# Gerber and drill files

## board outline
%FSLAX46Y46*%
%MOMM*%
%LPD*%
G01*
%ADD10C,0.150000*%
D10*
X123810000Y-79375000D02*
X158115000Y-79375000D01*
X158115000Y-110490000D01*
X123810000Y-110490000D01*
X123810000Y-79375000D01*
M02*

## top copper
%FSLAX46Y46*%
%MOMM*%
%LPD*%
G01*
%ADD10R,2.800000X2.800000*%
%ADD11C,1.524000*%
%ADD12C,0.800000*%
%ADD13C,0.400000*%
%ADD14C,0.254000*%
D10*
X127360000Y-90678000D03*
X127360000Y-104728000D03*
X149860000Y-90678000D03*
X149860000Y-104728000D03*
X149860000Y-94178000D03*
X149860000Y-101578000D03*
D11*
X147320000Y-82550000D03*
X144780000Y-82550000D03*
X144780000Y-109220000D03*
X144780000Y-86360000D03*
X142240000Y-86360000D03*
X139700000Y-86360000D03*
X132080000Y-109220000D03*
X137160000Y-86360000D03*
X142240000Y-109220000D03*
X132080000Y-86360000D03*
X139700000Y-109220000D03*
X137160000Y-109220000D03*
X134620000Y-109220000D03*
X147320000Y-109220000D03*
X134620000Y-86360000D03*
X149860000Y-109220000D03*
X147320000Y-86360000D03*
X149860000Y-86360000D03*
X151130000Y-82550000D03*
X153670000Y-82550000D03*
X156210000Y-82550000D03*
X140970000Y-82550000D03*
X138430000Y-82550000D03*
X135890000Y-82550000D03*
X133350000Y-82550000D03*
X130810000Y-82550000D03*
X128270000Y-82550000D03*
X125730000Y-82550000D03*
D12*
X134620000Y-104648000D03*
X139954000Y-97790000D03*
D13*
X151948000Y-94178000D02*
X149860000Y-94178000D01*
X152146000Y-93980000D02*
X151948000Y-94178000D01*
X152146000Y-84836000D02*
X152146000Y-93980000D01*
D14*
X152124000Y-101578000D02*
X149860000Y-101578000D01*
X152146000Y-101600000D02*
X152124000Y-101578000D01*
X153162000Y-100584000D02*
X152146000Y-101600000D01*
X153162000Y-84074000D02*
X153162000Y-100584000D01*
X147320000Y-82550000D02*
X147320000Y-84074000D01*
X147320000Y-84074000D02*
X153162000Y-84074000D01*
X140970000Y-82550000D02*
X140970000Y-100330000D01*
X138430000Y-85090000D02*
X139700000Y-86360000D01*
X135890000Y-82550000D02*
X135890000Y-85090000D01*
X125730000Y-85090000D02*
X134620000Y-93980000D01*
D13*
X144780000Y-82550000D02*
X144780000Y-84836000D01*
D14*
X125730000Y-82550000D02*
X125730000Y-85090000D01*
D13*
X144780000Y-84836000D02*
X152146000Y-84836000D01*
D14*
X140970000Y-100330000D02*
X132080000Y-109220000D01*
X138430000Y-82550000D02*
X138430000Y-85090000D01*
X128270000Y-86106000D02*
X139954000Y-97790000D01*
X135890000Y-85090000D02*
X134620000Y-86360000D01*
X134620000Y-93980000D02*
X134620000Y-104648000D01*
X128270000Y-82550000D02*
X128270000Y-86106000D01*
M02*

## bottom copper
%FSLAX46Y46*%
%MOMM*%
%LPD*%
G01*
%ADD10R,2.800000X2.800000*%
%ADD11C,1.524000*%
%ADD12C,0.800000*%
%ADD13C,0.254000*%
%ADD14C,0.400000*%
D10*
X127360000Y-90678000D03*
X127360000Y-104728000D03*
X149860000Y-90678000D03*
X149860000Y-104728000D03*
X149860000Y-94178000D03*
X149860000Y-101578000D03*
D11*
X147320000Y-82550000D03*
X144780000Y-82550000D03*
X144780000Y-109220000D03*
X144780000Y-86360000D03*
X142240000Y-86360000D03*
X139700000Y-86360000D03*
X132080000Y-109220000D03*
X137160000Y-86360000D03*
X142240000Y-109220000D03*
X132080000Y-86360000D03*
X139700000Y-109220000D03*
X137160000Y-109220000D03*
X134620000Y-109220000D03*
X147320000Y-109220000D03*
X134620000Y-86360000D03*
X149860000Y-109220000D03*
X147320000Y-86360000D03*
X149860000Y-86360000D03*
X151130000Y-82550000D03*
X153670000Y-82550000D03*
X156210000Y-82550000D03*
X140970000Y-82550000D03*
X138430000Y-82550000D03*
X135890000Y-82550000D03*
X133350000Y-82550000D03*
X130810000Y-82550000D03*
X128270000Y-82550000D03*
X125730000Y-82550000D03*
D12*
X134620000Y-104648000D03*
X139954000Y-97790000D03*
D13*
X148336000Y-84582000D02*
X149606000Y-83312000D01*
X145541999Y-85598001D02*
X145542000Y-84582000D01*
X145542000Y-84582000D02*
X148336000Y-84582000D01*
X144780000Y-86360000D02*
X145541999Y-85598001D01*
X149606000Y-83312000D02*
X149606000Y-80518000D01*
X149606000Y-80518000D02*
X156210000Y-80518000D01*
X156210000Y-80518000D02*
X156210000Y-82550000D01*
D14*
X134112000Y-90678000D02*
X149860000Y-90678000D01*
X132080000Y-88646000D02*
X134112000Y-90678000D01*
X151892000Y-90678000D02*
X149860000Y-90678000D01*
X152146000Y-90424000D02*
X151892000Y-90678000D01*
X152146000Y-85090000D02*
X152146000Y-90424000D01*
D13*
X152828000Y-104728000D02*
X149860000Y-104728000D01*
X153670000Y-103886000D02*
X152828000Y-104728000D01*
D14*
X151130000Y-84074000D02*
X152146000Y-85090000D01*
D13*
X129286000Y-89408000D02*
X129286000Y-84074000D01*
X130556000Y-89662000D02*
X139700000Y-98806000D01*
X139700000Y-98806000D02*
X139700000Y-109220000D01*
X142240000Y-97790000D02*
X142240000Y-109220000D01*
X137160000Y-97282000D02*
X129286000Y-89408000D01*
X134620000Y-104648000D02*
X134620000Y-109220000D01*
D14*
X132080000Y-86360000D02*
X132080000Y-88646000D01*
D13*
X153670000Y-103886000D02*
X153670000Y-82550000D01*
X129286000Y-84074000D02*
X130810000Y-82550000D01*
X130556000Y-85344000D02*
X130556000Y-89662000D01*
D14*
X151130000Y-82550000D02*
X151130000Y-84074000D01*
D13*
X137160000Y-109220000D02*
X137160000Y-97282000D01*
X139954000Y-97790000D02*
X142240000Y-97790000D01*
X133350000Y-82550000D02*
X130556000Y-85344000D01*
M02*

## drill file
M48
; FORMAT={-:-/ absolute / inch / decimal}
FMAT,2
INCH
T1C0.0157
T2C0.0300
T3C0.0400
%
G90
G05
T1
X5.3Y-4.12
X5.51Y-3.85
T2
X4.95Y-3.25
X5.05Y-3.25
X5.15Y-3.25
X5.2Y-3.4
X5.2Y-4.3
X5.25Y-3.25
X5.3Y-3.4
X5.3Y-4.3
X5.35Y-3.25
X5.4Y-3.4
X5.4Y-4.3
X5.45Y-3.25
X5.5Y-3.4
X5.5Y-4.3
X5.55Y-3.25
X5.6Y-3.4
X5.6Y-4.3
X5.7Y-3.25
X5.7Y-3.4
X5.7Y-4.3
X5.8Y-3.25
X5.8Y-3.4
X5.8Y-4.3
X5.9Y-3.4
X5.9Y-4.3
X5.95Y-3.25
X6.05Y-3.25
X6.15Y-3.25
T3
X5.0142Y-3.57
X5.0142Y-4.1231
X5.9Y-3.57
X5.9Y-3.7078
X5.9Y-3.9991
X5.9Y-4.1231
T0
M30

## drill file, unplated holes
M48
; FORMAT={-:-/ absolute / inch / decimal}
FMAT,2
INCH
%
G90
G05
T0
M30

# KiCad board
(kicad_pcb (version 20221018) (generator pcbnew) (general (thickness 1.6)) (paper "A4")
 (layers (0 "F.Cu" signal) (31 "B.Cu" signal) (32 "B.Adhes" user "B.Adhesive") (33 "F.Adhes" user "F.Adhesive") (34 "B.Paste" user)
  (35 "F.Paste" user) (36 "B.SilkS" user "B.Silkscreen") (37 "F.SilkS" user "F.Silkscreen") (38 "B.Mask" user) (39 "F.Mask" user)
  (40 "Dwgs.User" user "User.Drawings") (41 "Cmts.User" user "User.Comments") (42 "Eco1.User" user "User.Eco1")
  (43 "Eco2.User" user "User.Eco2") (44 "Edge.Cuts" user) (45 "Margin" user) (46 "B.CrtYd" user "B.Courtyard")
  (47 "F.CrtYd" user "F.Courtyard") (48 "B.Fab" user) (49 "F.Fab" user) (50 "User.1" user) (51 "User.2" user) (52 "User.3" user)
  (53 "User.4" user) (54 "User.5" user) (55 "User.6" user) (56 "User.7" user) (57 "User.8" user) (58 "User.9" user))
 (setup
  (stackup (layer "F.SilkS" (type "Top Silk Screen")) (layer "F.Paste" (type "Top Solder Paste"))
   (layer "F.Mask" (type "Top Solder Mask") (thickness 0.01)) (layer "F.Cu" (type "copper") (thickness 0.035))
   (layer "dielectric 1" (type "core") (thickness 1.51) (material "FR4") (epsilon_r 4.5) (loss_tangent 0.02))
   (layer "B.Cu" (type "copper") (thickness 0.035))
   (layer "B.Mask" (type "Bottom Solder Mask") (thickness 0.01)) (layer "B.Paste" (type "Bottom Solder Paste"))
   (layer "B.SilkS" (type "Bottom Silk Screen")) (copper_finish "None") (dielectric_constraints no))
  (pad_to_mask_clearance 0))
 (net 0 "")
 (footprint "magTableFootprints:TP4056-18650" (layer "F.Cu") (at 125.46 89.028)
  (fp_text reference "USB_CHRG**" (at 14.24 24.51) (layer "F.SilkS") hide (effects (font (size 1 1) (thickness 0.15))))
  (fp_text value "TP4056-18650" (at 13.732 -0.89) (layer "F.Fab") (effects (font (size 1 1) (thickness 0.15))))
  (pad "1" thru_hole rect (at 1.9 1.65) (size 2.8 2.8) (drill 1.016) (layers "*.Cu" "*.Mask"))
  (pad "2" thru_hole rect (at 1.9 15.7) (size 2.8 2.8) (drill 1.016) (layers "*.Cu" "*.Mask"))
  (pad "3" thru_hole rect (at 24.4 1.65) (size 2.8 2.8) (drill 1.016) (layers "*.Cu" "*.Mask"))
  (pad "4" thru_hole rect (at 24.4 15.7) (size 2.8 2.8) (drill 1.016) (layers "*.Cu" "*.Mask"))
  (pad "5" thru_hole rect (at 24.4 5.15) (size 2.8 2.8) (drill 1.016) (layers "*.Cu" "*.Mask"))
  (pad "6" thru_hole rect (at 24.4 12.55) (size 2.8 2.8) (drill 1.016) (layers "*.Cu" "*.Mask")))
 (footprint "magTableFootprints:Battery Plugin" (layer "F.Cu") (at 146.05 82.55 180)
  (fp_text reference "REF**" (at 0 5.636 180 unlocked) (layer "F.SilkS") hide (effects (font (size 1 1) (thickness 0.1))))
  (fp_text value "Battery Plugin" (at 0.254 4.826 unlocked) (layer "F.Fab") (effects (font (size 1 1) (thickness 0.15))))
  (pad "1" thru_hole circle (at -1.27 0 180) (size 1.524 1.524) (drill 0.762) (layers "*.Cu" "*.Mask"))
  (pad "2" thru_hole circle (at 1.27 0 180) (size 1.524 1.524) (drill 0.762) (layers "*.Cu" "*.Mask")))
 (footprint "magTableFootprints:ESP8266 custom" (layer "F.Cu") (at 140.97 97.79)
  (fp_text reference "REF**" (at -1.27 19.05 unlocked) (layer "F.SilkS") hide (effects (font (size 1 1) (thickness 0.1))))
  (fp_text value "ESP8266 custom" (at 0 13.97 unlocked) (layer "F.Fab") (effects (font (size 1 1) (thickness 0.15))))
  (pad "00" thru_hole circle (at 3.81 11.43) (size 1.524 1.524) (drill 0.762) (layers "*.Cu" "*.Mask"))
  (pad "1" thru_hole circle (at 3.81 -11.43) (size 1.524 1.524) (drill 0.762) (layers "*.Cu" "*.Mask"))
  (pad "2" thru_hole circle (at 1.27 -11.43) (size 1.524 1.524) (drill 0.762) (layers "*.Cu" "*.Mask"))
  (pad "3" thru_hole circle (at -1.27 -11.43) (size 1.524 1.524) (drill 0.762) (layers "*.Cu" "*.Mask"))
  (pad "3v" thru_hole circle (at -8.89 11.43) (size 1.524 1.524) (drill 0.762) (layers "*.Cu" "*.Mask"))
  (pad "4" thru_hole circle (at -3.81 -11.43) (size 1.524 1.524) (drill 0.762) (layers "*.Cu" "*.Mask"))
  (pad "5" thru_hole circle (at 1.27 11.43) (size 1.524 1.524) (drill 0.762) (layers "*.Cu" "*.Mask"))
  (pad "5V" thru_hole circle (at -8.89 -11.43) (size 1.524 1.524) (drill 0.762) (layers "*.Cu" "*.Mask"))
  (pad "6" thru_hole circle (at -1.27 11.43) (size 1.524 1.524) (drill 0.762) (layers "*.Cu" "*.Mask"))
  (pad "7" thru_hole circle (at -3.81 11.43) (size 1.524 1.524) (drill 0.762) (layers "*.Cu" "*.Mask"))
  (pad "8" thru_hole circle (at -6.35 11.43) (size 1.524 1.524) (drill 0.762) (layers "*.Cu" "*.Mask"))
  (pad "A0" thru_hole circle (at 6.35 11.43) (size 1.524 1.524) (drill 0.762) (layers "*.Cu" "*.Mask"))
  (pad "G" thru_hole circle (at -6.35 -11.43) (size 1.524 1.524) (drill 0.762) (layers "*.Cu" "*.Mask"))
  (pad "RST" thru_hole circle (at 8.89 11.43) (size 1.524 1.524) (drill 0.762) (layers "*.Cu" "*.Mask"))
  (pad "RX" thru_hole circle (at 6.35 -11.43) (size 1.524 1.524) (drill 0.762) (layers "*.Cu" "*.Mask"))
  (pad "TX" thru_hole circle (at 8.89 -11.43) (size 1.524 1.524) (drill 0.762) (layers "*.Cu" "*.Mask")))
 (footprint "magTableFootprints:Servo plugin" (layer "F.Cu") (at 153.67 82.55)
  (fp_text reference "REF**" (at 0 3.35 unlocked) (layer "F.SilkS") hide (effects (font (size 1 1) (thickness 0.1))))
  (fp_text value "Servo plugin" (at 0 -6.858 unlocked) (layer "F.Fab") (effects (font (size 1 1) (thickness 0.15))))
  (pad "1" thru_hole circle (at -2.54 0) (size 1.524 1.524) (drill 0.762) (layers "*.Cu" "*.Mask"))
  (pad "2" thru_hole circle (at 0 0) (size 1.524 1.524) (drill 0.762) (layers "*.Cu" "*.Mask"))
  (pad "3" thru_hole circle (at 2.54 0) (size 1.524 1.524) (drill 0.762) (layers "*.Cu" "*.Mask")))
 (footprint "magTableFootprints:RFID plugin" (layer "F.Cu") (at 133.35 82.55 180)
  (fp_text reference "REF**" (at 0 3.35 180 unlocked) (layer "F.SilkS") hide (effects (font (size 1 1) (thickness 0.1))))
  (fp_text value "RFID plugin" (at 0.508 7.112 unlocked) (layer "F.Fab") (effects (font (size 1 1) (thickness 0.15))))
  (pad "1" thru_hole circle (at -7.62 0 180) (size 1.524 1.524) (drill 0.762) (layers "*.Cu" "*.Mask"))
  (pad "2" thru_hole circle (at -5.08 0 180) (size 1.524 1.524) (drill 0.762) (layers "*.Cu" "*.Mask"))
  (pad "3" thru_hole circle (at -2.54 0 180) (size 1.524 1.524) (drill 0.762) (layers "*.Cu" "*.Mask"))
  (pad "4" thru_hole circle (at 0 0 180) (size 1.524 1.524) (drill 0.762) (layers "*.Cu" "*.Mask"))
  (pad "5" thru_hole circle (at 2.54 0 180) (size 1.524 1.524) (drill 0.762) (layers "*.Cu" "*.Mask"))
  (pad "6" thru_hole circle (at 5.08 0 270) (size 1.524 1.524) (drill 0.762) (layers "*.Cu" "*.Mask"))
  (pad "7" thru_hole circle (at 7.62 0 180) (size 1.524 1.524) (drill 0.762) (layers "*.Cu" "*.Mask")))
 (gr_rect (start 123.81 79.375) (end 158.115 110.49) (stroke (width 0.15) (type default)) (fill none) (layer "Edge.Cuts"))
 (segment (start 140.97 82.55) (end 140.97 100.33) (width 0.254) (layer "F.Cu") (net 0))
 (segment (start 138.43 85.09) (end 139.7 86.36) (width 0.254) (layer "F.Cu") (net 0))
 (segment (start 135.89 82.55) (end 135.89 85.09) (width 0.254) (layer "F.Cu") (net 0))
 (segment (start 152.124 101.578) (end 149.86 101.578) (width 0.254) (layer "F.Cu") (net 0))
 (segment (start 125.73 85.09) (end 134.62 93.98) (width 0.254) (layer "F.Cu") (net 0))
 (segment (start 152.146 84.836) (end 152.146 93.98) (width 0.4) (layer "F.Cu") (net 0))
 (segment (start 144.78 82.55) (end 144.78 84.836) (width 0.4) (layer "F.Cu") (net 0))
 (segment (start 151.948 94.178) (end 149.86 94.178) (width 0.4) (layer "F.Cu") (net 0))
 (segment (start 153.162 84.074) (end 153.162 100.584) (width 0.254) (layer "F.Cu") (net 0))
 (segment (start 125.73 82.55) (end 125.73 85.09) (width 0.254) (layer "F.Cu") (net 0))
 (segment (start 144.78 84.836) (end 152.146 84.836) (width 0.4) (layer "F.Cu") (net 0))
 (segment (start 140.97 100.33) (end 132.08 109.22) (width 0.254) (layer "F.Cu") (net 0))
 (segment (start 153.162 100.584) (end 152.146 101.6) (width 0.254) (layer "F.Cu") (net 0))
 (segment (start 152.146 101.6) (end 152.124 101.578) (width 0.254) (layer "F.Cu") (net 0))
 (segment (start 138.43 82.55) (end 138.43 85.09) (width 0.254) (layer "F.Cu") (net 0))
 (segment (start 128.27 86.106) (end 139.954 97.79) (width 0.254) (layer "F.Cu") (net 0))
 (segment (start 152.146 93.98) (end 151.948 94.178) (width 0.4) (layer "F.Cu") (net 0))
 (segment (start 135.89 85.09) (end 134.62 86.36) (width 0.254) (layer "F.Cu") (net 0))
 (segment (start 147.32 82.55) (end 147.32 84.074) (width 0.254) (layer "F.Cu") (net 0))
 (segment (start 147.32 84.074) (end 153.162 84.074) (width 0.254) (layer "F.Cu") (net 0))
 (segment (start 134.62 93.98) (end 134.62 104.648) (width 0.254) (layer "F.Cu") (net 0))
 (segment (start 128.27 82.55) (end 128.27 86.106) (width 0.254) (layer "F.Cu") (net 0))
 (via (at 134.62 104.648) (size 0.8) (drill 0.4) (layers "F.Cu" "B.Cu") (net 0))
 (via (at 139.954 97.79) (size 0.8) (drill 0.4) (layers "F.Cu" "B.Cu") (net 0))
 (segment (start 153.67 103.886) (end 152.828 104.728) (width 0.254) (layer "B.Cu") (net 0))
 (segment (start 156.21 80.518) (end 156.21 82.55) (width 0.254) (layer "B.Cu") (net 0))
 (segment (start 152.828 104.728) (end 149.86 104.728) (width 0.254) (layer "B.Cu") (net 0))
 (segment (start 151.892 90.678) (end 149.86 90.678) (width 0.4) (layer "B.Cu") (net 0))
 (segment (start 152.146 90.424) (end 151.892 90.678) (width 0.4) (layer "B.Cu") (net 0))
 (segment (start 132.08 88.646) (end 134.112 90.678) (width 0.4) (layer "B.Cu") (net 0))
 (segment (start 151.13 84.074) (end 152.146 85.09) (width 0.4) (layer "B.Cu") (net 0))
 (segment (start 129.286 89.408) (end 129.286 84.074) (width 0.254) (layer "B.Cu") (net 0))
 (segment (start 149.606 80.518) (end 156.21 80.518) (width 0.254) (layer "B.Cu") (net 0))
 (segment (start 130.556 89.662) (end 139.7 98.806) (width 0.254) (layer "B.Cu") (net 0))
 (segment (start 149.606 83.312) (end 149.606 80.518) (width 0.254) (layer "B.Cu") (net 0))
 (segment (start 139.7 98.806) (end 139.7 109.22) (width 0.254) (layer "B.Cu") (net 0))
 (segment (start 145.541999 85.598001) (end 145.542 84.582) (width 0.254) (layer "B.Cu") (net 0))
 (segment (start 142.24 97.79) (end 142.24 109.22) (width 0.254) (layer "B.Cu") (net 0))
 (segment (start 145.542 84.582) (end 148.336 84.582) (width 0.254) (layer "B.Cu") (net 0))
 (segment (start 137.16 97.282) (end 129.286 89.408) (width 0.254) (layer "B.Cu") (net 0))
 (segment (start 134.62 104.648) (end 134.62 109.22) (width 0.254) (layer "B.Cu") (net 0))
 (segment (start 144.78 86.36) (end 145.541999 85.598001) (width 0.254) (layer "B.Cu") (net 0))
 (segment (start 132.08 86.36) (end 132.08 88.646) (width 0.4) (layer "B.Cu") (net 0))
 (segment (start 148.336 84.582) (end 149.606 83.312) (width 0.254) (layer "B.Cu") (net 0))
 (segment (start 153.67 103.886) (end 153.67 82.55) (width 0.254) (layer "B.Cu") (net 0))
 (segment (start 129.286 84.074) (end 130.81 82.55) (width 0.254) (layer "B.Cu") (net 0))
 (segment (start 152.146 85.09) (end 152.146 90.424) (width 0.4) (layer "B.Cu") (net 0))
 (segment (start 130.556 85.344) (end 130.556 89.662) (width 0.254) (layer "B.Cu") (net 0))
 (segment (start 151.13 82.55) (end 151.13 84.074) (width 0.4) (layer "B.Cu") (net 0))
 (segment (start 137.16 109.22) (end 137.16 97.282) (width 0.254) (layer "B.Cu") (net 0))
 (segment (start 134.112 90.678) (end 149.86 90.678) (width 0.4) (layer "B.Cu") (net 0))
 (segment (start 139.954 97.79) (end 142.24 97.79) (width 0.254) (layer "B.Cu") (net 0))
 (segment (start 133.35 82.55) (end 130.556 85.344) (width 0.254) (layer "B.Cu") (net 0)))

